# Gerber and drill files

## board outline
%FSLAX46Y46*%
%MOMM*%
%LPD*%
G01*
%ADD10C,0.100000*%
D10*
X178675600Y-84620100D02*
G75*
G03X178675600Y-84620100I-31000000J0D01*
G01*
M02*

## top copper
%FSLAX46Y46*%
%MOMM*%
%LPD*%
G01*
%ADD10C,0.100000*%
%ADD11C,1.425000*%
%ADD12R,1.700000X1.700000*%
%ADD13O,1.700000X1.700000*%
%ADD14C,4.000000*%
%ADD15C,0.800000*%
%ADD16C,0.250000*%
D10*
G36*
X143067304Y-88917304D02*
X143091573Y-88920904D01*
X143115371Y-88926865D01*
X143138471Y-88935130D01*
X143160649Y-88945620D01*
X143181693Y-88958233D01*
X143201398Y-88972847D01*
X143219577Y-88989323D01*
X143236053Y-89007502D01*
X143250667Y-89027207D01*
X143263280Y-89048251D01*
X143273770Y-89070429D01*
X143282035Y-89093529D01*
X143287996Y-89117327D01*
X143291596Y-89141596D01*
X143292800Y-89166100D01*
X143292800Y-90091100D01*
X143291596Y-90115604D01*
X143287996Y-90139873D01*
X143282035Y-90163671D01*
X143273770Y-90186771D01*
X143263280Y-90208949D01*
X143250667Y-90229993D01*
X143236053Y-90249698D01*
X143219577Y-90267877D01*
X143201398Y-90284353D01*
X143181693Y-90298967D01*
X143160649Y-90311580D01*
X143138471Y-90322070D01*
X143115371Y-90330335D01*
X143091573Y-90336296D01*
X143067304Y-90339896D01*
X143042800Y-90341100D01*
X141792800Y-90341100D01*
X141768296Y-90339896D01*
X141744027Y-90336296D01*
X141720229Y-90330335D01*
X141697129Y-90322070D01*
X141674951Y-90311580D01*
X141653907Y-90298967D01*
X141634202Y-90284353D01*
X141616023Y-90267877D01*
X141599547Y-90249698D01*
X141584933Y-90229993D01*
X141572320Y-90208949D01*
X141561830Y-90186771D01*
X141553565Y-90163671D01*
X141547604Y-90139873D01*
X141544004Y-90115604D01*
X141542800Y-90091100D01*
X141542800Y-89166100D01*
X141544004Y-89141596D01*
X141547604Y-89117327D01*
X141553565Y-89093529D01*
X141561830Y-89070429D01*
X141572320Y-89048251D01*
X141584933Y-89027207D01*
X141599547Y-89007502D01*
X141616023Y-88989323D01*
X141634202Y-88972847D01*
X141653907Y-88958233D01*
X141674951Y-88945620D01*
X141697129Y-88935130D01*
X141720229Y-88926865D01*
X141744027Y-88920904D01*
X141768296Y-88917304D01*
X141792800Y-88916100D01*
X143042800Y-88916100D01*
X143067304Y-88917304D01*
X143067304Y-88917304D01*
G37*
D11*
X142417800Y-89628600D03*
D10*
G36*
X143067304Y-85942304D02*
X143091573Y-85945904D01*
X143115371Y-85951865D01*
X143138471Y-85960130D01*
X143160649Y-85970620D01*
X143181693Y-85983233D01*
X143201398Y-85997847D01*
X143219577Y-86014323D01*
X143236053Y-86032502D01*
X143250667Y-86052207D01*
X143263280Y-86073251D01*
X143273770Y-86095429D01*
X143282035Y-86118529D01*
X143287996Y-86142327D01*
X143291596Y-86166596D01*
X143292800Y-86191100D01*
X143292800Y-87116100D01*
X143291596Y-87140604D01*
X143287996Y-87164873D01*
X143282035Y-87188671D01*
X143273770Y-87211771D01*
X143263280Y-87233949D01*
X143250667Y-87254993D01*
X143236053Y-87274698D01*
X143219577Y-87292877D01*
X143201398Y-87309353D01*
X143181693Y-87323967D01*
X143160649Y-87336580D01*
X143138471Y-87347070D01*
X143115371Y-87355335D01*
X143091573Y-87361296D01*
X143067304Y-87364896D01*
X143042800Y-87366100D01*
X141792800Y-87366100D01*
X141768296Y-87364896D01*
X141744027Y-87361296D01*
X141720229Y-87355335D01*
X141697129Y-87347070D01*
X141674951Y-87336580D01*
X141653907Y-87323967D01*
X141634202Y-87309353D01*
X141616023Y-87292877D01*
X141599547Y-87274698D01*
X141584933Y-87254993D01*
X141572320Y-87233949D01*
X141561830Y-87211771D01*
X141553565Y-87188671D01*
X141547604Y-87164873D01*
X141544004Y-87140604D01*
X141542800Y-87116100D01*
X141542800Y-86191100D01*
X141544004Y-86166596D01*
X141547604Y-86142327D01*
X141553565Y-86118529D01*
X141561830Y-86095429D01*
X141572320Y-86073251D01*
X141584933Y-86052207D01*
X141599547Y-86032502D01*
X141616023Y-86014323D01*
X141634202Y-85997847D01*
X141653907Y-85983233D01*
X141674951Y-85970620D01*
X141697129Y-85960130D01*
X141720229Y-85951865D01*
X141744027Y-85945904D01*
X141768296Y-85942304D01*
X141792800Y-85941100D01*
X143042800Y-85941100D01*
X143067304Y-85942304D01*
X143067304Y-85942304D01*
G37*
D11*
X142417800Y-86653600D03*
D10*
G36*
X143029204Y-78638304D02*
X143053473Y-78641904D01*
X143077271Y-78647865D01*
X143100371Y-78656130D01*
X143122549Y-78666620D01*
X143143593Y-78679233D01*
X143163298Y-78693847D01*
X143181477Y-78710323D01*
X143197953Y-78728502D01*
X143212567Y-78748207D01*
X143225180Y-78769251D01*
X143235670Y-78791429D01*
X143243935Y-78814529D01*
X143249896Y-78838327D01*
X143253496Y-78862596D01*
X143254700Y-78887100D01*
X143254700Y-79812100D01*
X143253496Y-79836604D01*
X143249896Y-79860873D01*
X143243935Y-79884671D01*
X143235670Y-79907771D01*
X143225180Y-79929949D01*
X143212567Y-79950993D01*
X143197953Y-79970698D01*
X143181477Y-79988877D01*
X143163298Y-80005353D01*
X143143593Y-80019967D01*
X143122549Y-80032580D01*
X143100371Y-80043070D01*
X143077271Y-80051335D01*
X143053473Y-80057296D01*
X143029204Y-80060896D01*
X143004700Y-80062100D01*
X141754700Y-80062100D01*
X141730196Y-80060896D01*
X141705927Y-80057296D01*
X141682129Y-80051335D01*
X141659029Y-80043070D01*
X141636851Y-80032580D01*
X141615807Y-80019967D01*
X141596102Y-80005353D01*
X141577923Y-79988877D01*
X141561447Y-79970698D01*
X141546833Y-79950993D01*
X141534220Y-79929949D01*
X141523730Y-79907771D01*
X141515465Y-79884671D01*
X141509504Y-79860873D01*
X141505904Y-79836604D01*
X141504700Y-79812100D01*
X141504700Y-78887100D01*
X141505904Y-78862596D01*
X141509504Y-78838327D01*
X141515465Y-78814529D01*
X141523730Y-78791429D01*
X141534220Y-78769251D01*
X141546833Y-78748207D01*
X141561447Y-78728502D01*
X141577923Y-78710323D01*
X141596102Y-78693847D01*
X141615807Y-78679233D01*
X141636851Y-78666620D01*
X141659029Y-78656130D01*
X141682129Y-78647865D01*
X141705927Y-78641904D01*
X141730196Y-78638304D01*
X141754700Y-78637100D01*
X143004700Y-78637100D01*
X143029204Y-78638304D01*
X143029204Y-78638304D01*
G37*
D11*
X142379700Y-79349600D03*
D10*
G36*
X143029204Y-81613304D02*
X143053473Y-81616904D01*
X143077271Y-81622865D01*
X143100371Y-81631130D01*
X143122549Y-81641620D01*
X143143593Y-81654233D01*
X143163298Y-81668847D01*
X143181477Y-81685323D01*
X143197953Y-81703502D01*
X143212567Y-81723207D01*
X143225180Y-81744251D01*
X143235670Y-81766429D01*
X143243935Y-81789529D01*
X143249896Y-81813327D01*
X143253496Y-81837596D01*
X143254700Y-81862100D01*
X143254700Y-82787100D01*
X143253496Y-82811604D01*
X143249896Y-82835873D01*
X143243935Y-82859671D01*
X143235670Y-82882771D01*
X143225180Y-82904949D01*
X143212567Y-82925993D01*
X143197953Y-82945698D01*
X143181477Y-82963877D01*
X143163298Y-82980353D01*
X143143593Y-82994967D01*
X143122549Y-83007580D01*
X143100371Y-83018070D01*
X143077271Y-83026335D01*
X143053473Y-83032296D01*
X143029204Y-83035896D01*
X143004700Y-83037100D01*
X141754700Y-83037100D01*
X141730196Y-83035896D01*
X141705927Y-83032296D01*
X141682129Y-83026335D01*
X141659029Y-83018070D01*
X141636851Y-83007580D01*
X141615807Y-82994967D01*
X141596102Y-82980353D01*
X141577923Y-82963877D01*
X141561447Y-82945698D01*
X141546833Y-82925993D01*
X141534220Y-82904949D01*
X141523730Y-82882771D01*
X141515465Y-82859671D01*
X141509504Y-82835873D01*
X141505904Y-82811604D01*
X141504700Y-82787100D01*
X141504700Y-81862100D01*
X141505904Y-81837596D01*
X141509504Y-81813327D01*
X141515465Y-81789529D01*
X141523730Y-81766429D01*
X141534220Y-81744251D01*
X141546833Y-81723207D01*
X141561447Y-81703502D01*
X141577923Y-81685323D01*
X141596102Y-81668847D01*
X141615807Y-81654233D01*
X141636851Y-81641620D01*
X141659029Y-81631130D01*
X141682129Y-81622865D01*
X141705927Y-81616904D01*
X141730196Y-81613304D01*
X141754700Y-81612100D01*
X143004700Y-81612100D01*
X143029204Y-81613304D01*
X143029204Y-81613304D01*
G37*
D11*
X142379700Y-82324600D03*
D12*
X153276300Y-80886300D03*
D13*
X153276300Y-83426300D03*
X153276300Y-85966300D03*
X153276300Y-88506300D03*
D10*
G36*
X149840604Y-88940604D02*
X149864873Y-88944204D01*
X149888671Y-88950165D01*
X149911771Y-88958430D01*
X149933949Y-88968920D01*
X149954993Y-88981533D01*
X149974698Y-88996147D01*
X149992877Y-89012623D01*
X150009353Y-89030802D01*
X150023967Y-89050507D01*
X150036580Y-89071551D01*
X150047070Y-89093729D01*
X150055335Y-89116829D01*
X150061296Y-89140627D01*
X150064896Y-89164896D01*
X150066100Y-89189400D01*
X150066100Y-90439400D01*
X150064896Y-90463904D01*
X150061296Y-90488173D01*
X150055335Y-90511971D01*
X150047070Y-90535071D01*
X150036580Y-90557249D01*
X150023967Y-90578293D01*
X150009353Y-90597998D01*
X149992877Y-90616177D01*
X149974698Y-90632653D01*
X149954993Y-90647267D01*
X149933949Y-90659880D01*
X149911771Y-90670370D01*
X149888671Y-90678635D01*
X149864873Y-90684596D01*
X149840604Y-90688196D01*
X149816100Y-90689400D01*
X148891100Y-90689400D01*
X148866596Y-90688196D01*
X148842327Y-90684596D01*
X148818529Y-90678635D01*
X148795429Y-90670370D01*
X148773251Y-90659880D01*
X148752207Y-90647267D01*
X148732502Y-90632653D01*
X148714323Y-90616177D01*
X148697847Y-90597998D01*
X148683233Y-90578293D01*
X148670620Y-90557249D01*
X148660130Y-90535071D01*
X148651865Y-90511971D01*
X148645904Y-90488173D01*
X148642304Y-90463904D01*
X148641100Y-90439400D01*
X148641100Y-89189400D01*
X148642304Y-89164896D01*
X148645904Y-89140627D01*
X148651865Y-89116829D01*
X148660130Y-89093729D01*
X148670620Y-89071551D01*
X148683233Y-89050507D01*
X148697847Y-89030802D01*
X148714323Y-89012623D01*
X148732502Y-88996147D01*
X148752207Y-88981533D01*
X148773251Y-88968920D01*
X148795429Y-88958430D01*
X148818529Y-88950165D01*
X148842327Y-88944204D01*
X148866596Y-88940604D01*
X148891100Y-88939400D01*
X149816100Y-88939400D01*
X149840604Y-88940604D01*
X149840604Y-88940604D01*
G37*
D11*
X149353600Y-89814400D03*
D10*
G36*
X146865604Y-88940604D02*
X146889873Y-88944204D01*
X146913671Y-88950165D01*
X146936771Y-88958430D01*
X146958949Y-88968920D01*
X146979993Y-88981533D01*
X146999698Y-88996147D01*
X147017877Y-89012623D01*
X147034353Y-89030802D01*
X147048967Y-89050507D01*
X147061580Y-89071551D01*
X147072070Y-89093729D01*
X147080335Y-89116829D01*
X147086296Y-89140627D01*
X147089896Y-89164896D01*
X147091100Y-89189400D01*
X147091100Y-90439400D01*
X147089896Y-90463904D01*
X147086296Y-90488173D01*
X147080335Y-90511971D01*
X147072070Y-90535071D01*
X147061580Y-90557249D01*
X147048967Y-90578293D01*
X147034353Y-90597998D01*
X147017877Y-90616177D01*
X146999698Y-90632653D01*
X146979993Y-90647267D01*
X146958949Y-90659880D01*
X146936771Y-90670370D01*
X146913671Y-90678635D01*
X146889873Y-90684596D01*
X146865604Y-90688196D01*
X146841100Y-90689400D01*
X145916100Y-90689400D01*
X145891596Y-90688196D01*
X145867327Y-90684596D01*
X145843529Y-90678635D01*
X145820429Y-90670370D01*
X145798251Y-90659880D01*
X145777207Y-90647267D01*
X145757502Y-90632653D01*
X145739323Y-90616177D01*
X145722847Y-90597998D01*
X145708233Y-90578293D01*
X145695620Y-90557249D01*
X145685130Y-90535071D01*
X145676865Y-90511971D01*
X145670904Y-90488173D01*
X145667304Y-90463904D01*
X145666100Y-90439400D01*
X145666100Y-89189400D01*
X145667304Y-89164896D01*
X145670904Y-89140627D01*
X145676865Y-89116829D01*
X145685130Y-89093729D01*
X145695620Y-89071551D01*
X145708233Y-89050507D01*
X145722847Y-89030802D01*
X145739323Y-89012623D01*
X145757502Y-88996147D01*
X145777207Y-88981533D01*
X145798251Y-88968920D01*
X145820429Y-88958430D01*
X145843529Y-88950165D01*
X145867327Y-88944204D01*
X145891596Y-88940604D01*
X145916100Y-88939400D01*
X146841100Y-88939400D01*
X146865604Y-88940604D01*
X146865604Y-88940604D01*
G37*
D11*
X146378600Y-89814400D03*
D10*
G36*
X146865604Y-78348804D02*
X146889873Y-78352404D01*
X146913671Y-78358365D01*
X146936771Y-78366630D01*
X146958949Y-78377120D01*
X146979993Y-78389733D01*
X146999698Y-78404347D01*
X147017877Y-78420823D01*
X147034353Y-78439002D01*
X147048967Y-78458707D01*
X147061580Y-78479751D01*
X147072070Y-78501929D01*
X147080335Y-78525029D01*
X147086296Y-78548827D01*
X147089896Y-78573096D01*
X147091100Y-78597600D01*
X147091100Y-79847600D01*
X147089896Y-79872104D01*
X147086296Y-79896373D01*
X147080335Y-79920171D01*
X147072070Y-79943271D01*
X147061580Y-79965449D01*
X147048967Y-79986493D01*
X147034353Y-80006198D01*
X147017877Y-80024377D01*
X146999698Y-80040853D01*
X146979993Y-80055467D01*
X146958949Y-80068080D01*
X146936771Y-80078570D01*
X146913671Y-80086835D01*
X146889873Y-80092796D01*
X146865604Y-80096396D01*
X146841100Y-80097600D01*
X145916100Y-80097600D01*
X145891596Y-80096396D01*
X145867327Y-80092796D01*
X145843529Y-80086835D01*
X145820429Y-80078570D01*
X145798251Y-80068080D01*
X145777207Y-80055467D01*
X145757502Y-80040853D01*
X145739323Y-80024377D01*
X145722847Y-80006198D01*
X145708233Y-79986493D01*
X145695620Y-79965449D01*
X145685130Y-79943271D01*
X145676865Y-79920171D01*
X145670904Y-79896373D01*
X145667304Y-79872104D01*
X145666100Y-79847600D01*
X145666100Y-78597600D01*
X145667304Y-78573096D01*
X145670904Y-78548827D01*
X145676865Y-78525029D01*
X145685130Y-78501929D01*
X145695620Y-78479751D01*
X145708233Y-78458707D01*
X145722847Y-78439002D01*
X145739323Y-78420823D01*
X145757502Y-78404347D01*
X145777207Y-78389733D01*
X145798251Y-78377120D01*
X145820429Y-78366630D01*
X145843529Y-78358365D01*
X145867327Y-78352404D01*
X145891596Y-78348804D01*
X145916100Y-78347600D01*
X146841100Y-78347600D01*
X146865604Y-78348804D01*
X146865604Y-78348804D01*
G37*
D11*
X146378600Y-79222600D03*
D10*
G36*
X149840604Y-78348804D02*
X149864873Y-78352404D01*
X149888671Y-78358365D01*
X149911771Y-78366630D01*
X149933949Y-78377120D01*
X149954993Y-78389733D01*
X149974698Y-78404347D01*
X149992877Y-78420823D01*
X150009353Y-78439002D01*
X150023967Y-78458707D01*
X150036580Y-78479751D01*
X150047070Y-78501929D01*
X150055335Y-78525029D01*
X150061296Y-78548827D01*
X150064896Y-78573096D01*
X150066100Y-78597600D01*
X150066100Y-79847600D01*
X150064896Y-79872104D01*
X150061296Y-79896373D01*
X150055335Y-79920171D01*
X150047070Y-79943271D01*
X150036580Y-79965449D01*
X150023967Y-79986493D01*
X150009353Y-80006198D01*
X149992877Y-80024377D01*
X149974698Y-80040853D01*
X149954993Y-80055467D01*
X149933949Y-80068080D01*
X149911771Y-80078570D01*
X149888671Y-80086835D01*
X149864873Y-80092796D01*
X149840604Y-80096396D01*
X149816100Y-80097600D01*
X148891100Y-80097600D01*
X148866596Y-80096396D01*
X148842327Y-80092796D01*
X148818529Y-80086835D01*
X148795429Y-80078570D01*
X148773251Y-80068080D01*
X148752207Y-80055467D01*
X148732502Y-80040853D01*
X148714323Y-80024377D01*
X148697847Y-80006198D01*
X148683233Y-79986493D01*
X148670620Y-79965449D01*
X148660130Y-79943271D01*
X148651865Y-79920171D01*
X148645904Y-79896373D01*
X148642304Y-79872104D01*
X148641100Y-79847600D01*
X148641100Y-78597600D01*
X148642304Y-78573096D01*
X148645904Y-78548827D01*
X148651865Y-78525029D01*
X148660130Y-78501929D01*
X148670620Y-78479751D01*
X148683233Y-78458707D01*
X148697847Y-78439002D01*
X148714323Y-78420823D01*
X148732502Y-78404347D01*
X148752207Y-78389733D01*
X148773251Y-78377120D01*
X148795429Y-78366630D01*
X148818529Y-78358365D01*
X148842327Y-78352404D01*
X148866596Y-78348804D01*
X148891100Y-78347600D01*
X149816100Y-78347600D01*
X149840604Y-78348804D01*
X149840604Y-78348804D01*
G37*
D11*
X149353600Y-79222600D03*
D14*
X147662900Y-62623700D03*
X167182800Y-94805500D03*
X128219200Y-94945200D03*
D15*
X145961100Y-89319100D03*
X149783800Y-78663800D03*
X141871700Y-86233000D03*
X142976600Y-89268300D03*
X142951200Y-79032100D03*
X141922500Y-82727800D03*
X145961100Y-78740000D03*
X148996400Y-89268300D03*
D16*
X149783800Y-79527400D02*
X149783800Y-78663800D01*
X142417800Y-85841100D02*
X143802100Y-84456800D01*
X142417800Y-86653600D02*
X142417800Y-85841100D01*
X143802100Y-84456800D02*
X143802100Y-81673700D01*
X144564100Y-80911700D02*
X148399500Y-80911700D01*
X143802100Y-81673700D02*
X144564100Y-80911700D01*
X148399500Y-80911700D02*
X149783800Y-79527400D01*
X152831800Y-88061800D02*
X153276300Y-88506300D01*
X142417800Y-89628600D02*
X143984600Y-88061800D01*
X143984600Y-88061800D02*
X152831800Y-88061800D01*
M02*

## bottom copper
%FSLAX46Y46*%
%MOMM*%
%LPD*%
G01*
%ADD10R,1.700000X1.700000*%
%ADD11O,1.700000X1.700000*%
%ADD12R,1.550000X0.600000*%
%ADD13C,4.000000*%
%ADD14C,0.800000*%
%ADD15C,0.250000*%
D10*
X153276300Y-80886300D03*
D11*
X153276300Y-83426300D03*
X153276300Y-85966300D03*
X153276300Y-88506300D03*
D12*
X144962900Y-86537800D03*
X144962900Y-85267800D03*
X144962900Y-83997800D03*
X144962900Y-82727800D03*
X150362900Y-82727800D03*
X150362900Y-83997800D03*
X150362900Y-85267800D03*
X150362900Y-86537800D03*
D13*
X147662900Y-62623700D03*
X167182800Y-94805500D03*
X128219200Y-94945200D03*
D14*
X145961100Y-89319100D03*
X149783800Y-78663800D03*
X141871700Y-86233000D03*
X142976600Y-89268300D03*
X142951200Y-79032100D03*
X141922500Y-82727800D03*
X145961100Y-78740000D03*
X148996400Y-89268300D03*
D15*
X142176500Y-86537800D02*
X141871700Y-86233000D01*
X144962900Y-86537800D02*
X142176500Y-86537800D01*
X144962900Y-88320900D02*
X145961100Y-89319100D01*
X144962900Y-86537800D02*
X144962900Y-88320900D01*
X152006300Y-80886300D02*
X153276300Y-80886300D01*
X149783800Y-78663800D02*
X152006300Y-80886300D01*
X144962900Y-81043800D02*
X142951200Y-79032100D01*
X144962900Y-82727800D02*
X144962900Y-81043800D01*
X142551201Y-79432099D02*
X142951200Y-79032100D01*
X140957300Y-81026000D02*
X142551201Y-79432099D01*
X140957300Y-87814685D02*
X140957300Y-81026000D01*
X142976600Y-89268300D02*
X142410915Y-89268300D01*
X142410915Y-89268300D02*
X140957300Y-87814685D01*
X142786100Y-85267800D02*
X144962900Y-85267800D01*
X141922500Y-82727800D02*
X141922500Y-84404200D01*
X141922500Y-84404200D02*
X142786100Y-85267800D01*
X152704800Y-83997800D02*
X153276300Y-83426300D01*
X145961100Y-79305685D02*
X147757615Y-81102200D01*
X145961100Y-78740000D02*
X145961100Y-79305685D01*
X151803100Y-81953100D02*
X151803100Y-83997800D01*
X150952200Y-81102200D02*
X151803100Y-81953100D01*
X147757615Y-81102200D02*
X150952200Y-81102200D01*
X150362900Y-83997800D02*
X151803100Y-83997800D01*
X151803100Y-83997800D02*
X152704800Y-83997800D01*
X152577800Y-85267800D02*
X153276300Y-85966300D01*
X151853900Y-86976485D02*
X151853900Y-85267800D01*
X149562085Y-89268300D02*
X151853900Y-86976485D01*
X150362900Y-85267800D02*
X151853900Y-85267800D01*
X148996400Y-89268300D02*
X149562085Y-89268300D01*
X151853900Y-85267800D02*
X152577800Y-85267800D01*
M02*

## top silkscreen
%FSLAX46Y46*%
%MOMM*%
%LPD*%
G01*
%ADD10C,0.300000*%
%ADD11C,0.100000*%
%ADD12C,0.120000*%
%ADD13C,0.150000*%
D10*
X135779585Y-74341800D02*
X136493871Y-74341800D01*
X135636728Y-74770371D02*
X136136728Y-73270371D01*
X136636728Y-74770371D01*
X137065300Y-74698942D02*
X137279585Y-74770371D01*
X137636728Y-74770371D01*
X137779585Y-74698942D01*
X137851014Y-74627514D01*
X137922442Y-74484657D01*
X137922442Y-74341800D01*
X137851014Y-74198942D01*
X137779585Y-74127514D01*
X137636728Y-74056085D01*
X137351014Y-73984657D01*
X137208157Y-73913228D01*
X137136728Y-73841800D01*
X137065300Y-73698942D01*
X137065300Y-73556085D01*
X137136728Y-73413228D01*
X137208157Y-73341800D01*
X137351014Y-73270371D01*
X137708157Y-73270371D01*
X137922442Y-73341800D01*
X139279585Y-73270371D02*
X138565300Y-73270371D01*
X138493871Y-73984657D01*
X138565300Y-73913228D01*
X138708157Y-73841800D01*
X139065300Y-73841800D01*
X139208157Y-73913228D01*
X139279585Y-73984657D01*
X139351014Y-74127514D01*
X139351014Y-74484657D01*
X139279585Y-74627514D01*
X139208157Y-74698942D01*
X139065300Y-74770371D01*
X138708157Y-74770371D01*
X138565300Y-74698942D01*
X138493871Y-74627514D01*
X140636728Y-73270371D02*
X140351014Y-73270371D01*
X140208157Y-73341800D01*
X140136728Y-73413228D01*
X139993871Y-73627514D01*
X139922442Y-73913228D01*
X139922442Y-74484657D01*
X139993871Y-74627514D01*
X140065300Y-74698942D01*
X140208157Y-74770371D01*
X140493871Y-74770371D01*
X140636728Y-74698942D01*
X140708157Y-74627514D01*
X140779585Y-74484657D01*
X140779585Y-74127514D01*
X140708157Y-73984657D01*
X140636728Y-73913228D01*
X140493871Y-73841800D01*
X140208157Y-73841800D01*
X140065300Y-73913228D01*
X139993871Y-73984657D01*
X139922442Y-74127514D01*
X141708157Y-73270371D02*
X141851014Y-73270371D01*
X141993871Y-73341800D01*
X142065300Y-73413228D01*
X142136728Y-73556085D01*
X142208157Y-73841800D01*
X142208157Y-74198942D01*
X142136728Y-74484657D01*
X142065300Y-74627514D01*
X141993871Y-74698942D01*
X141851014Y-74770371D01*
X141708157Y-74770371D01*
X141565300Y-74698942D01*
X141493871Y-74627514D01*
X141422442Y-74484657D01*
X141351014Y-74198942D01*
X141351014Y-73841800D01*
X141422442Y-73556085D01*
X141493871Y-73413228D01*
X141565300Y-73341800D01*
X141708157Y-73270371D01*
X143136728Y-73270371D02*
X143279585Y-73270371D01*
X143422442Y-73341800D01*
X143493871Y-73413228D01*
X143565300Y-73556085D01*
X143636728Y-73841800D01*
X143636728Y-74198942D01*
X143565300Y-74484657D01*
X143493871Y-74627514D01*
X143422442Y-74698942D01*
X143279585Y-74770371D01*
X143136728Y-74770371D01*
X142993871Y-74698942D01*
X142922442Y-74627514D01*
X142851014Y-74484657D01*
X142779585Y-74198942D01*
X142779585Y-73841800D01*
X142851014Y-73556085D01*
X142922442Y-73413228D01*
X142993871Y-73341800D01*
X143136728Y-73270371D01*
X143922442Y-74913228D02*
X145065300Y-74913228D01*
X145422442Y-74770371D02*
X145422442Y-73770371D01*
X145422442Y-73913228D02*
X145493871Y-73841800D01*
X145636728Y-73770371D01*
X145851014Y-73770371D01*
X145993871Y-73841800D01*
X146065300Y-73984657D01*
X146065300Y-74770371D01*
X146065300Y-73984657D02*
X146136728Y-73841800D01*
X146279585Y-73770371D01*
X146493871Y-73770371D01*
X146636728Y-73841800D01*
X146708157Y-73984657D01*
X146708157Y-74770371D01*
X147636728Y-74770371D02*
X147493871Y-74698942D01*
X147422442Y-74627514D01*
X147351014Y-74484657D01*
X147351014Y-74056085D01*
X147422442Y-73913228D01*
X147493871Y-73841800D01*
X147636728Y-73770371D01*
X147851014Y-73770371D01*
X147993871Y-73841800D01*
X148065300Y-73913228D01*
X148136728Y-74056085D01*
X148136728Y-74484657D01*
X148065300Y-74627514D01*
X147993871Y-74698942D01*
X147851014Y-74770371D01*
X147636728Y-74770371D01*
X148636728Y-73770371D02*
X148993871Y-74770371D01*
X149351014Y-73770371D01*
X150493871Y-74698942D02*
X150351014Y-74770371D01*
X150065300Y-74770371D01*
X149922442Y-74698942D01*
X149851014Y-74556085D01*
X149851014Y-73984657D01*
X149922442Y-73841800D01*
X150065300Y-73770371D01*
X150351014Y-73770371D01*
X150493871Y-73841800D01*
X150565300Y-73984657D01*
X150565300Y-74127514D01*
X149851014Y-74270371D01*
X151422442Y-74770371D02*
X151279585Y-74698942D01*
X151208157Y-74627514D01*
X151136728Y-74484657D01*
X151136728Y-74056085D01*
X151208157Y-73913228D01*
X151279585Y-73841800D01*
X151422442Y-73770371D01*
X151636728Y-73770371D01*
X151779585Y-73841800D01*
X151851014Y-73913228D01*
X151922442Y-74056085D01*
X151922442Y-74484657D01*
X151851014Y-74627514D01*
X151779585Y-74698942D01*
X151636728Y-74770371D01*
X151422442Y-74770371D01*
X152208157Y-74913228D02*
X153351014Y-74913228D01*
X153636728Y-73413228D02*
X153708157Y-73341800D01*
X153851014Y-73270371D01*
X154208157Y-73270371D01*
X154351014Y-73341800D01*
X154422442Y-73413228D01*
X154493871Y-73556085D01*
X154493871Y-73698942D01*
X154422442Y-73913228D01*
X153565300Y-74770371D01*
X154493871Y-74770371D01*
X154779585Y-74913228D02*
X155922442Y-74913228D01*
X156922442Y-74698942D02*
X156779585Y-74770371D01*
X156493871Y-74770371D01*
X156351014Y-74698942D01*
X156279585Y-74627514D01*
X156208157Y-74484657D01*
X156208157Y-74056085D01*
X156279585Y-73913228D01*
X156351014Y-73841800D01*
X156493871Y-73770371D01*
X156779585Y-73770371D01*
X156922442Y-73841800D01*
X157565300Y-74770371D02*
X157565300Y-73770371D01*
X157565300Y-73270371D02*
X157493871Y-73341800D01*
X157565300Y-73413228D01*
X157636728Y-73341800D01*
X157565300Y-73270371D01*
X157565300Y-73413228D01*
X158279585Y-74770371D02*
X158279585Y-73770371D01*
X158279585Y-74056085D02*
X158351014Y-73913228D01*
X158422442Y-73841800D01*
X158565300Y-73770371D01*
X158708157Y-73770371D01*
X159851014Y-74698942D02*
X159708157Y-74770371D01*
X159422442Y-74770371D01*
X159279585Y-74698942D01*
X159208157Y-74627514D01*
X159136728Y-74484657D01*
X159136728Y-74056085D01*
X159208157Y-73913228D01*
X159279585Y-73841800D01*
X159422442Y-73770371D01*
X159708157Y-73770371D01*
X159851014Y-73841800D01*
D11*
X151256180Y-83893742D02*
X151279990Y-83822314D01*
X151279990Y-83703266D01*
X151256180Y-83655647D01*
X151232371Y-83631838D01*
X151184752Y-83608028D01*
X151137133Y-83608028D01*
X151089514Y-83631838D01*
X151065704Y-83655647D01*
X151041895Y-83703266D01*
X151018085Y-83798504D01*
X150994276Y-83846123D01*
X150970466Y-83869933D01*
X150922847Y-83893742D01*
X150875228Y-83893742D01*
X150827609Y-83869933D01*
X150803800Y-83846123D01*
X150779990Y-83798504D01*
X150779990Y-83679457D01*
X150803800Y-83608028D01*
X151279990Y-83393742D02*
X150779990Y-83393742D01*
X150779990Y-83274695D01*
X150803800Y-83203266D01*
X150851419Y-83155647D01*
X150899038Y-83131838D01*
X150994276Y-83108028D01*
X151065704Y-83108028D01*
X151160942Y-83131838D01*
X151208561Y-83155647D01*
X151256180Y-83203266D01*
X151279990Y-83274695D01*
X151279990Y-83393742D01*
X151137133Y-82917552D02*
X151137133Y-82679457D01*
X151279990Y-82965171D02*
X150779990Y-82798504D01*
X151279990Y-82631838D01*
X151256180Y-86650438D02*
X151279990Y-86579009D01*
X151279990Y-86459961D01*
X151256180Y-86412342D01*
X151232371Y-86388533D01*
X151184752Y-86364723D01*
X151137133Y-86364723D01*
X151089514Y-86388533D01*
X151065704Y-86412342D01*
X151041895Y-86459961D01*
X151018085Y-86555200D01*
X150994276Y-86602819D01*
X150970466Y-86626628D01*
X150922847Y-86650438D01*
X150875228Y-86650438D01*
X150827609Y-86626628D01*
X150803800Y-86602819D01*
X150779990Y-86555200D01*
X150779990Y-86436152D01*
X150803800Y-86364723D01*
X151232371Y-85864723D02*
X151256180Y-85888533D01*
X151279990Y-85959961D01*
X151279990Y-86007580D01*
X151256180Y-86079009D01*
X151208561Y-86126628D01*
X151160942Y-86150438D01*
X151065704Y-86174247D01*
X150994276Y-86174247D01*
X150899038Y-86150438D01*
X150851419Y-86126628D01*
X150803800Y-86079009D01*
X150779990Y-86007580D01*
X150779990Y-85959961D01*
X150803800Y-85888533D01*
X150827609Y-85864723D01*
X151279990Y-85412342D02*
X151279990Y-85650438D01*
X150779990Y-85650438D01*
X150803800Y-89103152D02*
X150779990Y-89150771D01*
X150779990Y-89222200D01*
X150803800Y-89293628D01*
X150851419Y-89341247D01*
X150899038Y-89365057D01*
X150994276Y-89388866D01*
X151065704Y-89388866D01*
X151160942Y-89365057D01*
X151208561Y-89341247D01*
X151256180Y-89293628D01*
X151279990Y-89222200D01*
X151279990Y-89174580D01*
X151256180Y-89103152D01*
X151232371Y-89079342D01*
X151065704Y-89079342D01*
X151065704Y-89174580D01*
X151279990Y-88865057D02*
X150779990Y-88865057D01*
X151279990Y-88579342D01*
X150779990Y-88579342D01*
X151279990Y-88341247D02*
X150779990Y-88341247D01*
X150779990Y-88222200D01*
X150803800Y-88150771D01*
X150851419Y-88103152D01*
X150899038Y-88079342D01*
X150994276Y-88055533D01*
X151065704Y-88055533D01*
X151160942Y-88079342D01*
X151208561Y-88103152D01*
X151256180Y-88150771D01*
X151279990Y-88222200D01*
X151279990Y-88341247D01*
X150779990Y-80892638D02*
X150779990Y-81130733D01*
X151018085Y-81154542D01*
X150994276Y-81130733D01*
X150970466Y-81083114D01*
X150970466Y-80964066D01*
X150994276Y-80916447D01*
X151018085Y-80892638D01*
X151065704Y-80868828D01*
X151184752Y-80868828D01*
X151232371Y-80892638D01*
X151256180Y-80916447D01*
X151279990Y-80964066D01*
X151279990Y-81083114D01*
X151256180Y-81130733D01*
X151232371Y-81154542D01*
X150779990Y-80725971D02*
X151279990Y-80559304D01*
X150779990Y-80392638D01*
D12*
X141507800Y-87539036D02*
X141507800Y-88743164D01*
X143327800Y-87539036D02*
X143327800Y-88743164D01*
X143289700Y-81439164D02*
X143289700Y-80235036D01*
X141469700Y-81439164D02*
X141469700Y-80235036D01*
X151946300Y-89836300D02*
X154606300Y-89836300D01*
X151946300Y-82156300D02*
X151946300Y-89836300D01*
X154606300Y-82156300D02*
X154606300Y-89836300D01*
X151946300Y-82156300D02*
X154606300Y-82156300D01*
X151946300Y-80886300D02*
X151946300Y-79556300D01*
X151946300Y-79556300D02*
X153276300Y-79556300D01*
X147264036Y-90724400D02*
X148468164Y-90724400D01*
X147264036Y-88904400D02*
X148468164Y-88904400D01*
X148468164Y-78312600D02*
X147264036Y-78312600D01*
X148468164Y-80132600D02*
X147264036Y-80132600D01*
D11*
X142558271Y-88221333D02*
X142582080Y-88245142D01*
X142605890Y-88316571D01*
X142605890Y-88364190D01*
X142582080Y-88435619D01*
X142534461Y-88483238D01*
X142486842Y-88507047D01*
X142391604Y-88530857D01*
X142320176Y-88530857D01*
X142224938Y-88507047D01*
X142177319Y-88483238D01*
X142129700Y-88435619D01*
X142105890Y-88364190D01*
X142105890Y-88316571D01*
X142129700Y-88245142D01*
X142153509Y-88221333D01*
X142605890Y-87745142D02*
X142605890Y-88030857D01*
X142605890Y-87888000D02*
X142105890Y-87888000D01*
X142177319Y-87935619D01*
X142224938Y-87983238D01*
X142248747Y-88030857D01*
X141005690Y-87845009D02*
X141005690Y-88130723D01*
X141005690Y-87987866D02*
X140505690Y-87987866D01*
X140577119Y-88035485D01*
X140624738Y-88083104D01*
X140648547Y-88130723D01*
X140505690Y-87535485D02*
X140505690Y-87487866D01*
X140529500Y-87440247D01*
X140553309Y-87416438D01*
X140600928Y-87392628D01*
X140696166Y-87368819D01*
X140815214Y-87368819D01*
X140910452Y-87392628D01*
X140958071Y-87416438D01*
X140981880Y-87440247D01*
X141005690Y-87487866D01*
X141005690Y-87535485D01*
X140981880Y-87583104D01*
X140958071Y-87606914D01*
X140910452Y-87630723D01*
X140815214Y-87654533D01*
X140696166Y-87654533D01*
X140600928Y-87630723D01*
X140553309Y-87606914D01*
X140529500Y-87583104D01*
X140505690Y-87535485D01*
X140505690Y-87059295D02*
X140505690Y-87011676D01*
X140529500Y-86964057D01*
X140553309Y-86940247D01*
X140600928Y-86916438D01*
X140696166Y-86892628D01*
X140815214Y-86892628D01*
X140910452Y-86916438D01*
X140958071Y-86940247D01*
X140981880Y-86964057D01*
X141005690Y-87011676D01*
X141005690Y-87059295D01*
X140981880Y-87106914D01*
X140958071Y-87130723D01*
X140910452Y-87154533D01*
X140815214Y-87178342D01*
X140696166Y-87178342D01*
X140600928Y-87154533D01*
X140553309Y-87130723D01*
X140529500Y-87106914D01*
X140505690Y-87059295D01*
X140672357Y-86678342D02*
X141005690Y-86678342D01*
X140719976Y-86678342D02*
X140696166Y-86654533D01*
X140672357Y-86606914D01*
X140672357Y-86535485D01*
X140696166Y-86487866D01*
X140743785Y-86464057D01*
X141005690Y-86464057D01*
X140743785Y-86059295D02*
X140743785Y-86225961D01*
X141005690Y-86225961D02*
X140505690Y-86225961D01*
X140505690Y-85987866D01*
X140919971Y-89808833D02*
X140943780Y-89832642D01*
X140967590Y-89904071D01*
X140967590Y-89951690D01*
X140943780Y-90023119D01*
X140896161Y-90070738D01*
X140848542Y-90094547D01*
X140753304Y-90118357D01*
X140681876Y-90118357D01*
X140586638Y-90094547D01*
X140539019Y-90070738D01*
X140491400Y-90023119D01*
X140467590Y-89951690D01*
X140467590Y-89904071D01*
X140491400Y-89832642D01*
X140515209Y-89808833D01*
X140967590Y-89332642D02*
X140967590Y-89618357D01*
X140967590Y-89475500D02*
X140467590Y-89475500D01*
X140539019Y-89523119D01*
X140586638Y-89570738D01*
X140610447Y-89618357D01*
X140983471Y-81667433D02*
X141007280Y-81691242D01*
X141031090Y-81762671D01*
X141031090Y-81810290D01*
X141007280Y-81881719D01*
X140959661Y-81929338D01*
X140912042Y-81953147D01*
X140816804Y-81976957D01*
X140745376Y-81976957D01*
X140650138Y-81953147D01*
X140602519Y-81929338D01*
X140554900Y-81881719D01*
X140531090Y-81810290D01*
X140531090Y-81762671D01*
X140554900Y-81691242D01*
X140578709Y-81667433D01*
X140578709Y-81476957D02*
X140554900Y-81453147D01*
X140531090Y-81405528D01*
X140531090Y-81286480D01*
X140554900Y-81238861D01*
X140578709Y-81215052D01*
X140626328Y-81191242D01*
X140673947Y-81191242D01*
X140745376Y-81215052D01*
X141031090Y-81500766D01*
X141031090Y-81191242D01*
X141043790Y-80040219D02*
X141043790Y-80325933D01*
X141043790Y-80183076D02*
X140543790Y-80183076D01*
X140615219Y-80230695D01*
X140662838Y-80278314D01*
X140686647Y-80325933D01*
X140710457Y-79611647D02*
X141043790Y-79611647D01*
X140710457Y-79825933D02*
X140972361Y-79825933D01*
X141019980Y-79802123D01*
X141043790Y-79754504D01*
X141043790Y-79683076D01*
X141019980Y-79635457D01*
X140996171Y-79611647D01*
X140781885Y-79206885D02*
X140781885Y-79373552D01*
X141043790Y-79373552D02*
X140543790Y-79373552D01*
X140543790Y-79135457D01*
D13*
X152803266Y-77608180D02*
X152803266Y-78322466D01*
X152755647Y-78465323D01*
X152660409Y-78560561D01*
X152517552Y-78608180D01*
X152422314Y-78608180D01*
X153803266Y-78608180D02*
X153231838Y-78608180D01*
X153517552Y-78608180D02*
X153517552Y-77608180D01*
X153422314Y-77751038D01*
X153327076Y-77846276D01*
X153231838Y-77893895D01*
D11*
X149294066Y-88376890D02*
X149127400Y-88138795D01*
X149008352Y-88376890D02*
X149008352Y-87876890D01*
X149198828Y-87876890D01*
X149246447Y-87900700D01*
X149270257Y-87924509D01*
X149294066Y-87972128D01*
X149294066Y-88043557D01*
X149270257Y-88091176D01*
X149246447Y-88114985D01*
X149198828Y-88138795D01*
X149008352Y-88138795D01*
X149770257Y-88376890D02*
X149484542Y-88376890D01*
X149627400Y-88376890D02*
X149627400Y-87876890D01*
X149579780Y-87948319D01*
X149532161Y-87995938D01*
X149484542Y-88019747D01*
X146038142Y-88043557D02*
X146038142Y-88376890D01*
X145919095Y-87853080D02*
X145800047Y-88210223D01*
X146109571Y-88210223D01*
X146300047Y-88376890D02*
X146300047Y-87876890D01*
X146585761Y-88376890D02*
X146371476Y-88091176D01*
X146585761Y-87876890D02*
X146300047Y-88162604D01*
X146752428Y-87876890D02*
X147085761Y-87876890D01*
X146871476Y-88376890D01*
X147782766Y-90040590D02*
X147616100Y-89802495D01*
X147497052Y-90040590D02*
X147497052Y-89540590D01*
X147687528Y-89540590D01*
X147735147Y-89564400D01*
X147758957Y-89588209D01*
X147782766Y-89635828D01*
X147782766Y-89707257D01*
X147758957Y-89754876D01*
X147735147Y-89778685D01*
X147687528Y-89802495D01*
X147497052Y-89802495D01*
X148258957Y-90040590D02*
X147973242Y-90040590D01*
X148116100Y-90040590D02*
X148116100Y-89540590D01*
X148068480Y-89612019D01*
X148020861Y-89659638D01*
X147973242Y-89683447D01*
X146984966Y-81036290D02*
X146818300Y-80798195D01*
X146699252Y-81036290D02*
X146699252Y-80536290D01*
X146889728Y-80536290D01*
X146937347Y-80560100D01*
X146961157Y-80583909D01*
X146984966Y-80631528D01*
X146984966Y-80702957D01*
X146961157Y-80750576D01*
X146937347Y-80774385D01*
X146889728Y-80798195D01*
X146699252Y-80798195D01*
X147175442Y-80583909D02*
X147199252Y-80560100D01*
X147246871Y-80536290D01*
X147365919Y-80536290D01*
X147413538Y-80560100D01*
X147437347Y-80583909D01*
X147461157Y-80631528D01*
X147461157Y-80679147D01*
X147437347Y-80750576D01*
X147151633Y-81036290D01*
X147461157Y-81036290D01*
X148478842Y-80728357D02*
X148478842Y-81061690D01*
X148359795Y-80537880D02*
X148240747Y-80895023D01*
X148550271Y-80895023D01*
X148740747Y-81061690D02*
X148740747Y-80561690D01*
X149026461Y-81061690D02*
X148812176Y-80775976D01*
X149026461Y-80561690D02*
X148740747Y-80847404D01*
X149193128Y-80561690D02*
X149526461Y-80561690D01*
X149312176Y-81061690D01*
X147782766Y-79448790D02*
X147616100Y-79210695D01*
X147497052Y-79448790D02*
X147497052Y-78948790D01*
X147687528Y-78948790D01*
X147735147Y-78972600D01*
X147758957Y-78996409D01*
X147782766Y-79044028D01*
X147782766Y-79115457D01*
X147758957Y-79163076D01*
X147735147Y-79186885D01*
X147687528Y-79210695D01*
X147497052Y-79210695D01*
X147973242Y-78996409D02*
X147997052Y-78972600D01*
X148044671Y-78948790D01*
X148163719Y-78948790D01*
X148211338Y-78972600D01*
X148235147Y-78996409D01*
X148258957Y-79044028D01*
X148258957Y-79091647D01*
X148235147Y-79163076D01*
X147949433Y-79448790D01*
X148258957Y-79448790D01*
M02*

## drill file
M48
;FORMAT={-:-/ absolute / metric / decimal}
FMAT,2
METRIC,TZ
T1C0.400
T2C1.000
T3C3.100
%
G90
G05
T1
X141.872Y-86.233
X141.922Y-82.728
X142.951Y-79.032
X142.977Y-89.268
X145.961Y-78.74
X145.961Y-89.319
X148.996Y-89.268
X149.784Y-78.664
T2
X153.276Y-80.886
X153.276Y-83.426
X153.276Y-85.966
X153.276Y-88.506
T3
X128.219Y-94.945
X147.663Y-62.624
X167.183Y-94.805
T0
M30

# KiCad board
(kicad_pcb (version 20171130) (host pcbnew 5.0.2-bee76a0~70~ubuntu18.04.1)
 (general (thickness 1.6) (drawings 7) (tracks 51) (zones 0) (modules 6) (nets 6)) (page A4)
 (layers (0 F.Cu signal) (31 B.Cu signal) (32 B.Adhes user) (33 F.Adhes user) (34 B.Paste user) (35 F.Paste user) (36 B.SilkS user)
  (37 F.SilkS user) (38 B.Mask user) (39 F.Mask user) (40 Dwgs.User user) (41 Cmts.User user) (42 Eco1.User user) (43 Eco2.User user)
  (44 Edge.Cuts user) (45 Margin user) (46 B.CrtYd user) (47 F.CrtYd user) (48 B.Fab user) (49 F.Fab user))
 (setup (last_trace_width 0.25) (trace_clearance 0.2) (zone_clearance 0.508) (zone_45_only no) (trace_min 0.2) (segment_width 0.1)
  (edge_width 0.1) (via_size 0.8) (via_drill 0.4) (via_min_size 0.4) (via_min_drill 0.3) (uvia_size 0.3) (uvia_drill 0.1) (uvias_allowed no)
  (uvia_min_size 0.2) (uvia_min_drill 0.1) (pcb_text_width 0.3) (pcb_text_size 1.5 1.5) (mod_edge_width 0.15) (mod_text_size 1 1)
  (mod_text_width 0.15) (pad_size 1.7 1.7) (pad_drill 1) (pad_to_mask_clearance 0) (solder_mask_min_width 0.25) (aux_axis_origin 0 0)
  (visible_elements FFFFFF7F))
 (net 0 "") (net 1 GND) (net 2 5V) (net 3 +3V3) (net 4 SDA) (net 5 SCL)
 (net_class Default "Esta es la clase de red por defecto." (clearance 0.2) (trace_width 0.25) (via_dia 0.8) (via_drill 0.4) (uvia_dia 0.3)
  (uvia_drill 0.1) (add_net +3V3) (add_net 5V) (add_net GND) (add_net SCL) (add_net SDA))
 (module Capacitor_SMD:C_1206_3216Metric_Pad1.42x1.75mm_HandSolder (layer F.Cu) (at 142.4178 88.1411 270)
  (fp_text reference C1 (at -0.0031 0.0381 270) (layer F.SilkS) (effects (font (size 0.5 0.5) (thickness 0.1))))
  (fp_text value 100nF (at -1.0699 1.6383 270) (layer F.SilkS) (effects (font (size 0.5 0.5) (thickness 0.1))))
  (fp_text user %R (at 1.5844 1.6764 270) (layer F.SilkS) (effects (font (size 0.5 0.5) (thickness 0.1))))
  (fp_line (start -0.602064 0.91) (end 0.602064 0.91) (layer F.SilkS) (width 0.12))
  (fp_line (start -0.602064 -0.91) (end 0.602064 -0.91) (layer F.SilkS) (width 0.12))
  (pad 2 smd roundrect (at 1.4875 0 270) (size 1.425 1.75) (layers F.Cu F.Paste F.Mask) (roundrect_rratio 0.175439) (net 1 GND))
  (pad 1 smd roundrect (at -1.4875 0 270) (size 1.425 1.75) (layers F.Cu F.Paste F.Mask) (roundrect_rratio 0.175439) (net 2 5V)))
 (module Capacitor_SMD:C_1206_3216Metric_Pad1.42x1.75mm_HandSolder (layer F.Cu) (at 142.3797 80.8371 90)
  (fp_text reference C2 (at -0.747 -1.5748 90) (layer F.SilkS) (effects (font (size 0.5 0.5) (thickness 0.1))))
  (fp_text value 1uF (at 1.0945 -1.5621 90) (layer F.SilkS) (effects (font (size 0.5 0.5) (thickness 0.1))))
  (fp_line (start -0.602064 0.91) (end 0.602064 0.91) (layer F.SilkS) (width 0.12))
  (fp_line (start -0.602064 -0.91) (end 0.602064 -0.91) (layer F.SilkS) (width 0.12))
  (pad 2 smd roundrect (at 1.4875 0 90) (size 1.425 1.75) (layers F.Cu F.Paste F.Mask) (roundrect_rratio 0.175439) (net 1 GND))
  (pad 1 smd roundrect (at -1.4875 0 90) (size 1.425 1.75) (layers F.Cu F.Paste F.Mask) (roundrect_rratio 0.175439) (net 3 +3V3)))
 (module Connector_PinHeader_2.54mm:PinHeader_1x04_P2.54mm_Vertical (layer F.Cu) (at 153.2763 80.8863)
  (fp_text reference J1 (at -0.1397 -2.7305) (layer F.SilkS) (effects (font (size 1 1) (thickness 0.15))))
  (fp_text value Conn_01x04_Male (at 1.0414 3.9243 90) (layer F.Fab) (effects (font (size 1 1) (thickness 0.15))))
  (fp_line (start -1.33 8.95) (end 1.33 8.95) (layer F.SilkS) (width 0.12))
  (fp_line (start -1.33 1.27) (end -1.33 8.95) (layer F.SilkS) (width 0.12))
  (fp_line (start 1.33 1.27) (end 1.33 8.95) (layer F.SilkS) (width 0.12))
  (fp_line (start -1.33 1.27) (end 1.33 1.27) (layer F.SilkS) (width 0.12))
  (fp_line (start -1.33 0) (end -1.33 -1.33) (layer F.SilkS) (width 0.12))
  (fp_line (start -1.33 -1.33) (end 0 -1.33) (layer F.SilkS) (width 0.12))
  (pad 1 thru_hole rect (at 0 0) (size 1.7 1.7) (drill 1) (layers *.Cu *.Mask) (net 2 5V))
  (pad 2 thru_hole oval (at 0 2.54) (size 1.7 1.7) (drill 1) (layers *.Cu *.Mask) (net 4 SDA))
  (pad 3 thru_hole oval (at 0 5.08) (size 1.7 1.7) (drill 1) (layers *.Cu *.Mask) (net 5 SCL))
  (pad 4 thru_hole oval (at 0 7.62) (size 1.7 1.7) (drill 1) (layers *.Cu *.Mask) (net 1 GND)))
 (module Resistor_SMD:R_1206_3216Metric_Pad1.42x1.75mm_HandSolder (layer F.Cu) (at 147.8661 89.8144)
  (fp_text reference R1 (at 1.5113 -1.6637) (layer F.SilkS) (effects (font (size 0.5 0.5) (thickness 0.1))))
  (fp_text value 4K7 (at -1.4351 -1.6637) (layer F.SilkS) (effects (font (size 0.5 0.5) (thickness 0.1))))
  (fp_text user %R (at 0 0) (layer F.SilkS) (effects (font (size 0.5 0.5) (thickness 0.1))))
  (fp_line (start -0.602064 0.91) (end 0.602064 0.91) (layer F.SilkS) (width 0.12))
  (fp_line (start -0.602064 -0.91) (end 0.602064 -0.91) (layer F.SilkS) (width 0.12))
  (pad 2 smd roundrect (at 1.4875 0) (size 1.425 1.75) (layers F.Cu F.Paste F.Mask) (roundrect_rratio 0.175439) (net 5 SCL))
  (pad 1 smd roundrect (at -1.4875 0) (size 1.425 1.75) (layers F.Cu F.Paste F.Mask) (roundrect_rratio 0.175439) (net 2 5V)))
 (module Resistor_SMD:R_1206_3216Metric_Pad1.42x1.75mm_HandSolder (layer F.Cu) (at 147.8661 79.2226 180)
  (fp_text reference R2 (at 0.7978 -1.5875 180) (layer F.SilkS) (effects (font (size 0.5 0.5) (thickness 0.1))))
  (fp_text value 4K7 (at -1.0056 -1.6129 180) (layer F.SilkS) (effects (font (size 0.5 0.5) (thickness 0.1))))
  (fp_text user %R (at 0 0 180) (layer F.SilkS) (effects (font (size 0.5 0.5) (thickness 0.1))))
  (fp_line (start -0.602064 0.91) (end 0.602064 0.91) (layer F.SilkS) (width 0.12))
  (fp_line (start -0.602064 -0.91) (end 0.602064 -0.91) (layer F.SilkS) (width 0.12))
  (pad 2 smd roundrect (at 1.4875 0 180) (size 1.425 1.75) (layers F.Cu F.Paste F.Mask) (roundrect_rratio 0.175439) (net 4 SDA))
  (pad 1 smd roundrect (at -1.4875 0 180) (size 1.425 1.75) (layers F.Cu F.Paste F.Mask) (roundrect_rratio 0.175439) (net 2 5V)))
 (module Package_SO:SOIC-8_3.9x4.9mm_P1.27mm (layer B.Cu) (at 147.6629 84.6328)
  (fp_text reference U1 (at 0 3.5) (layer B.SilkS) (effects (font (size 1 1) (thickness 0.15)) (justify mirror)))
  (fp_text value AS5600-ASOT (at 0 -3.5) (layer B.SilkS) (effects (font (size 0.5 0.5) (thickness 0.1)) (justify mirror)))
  (pad 1 smd rect (at -2.7 1.905) (size 1.55 0.6) (layers B.Cu B.Paste B.Mask) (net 2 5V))
  (pad 2 smd rect (at -2.7 0.635) (size 1.55 0.6) (layers B.Cu B.Paste B.Mask) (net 3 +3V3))
  (pad 3 smd rect (at -2.7 -0.635) (size 1.55 0.6) (layers B.Cu B.Paste B.Mask))
  (pad 4 smd rect (at -2.7 -1.905) (size 1.55 0.6) (layers B.Cu B.Paste B.Mask) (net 1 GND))
  (pad 5 smd rect (at 2.7 -1.905) (size 1.55 0.6) (layers B.Cu B.Paste B.Mask))
  (pad 6 smd rect (at 2.7 -0.635) (size 1.55 0.6) (layers B.Cu B.Paste B.Mask) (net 4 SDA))
  (pad 7 smd rect (at 2.7 0.635) (size 1.55 0.6) (layers B.Cu B.Paste B.Mask) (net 5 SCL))
  (pad 8 smd rect (at 2.7 1.905) (size 1.55 0.6) (layers B.Cu B.Paste B.Mask)))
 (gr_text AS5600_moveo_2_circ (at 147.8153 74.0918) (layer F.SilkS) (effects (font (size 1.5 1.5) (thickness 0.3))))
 (gr_circle (center 147.6756 84.6201) (end 178.6756 84.6201) (layer Edge.Cuts) (width 0.1))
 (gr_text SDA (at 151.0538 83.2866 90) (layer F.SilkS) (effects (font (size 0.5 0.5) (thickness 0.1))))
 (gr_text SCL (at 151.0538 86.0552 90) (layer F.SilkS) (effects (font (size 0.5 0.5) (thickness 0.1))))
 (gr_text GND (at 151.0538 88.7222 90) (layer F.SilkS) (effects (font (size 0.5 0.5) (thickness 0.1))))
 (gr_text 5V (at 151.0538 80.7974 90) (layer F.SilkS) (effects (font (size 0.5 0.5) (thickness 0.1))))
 (via (at 147.6629 62.6237) (size 4) (drill 3.1) (layers F.Cu B.Cu) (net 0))
 (via (at 167.1828 94.8055) (size 4) (drill 3.1) (layers F.Cu B.Cu) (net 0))
 (via (at 128.2192 94.9452) (size 4) (drill 3.1) (layers F.Cu B.Cu) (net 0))
 (via (at 145.9611 89.3191) (size 0.8) (drill 0.4) (layers F.Cu B.Cu) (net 2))
 (via (at 149.7838 78.6638) (size 0.8) (drill 0.4) (layers F.Cu B.Cu) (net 2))
 (via (at 141.8717 86.233) (size 0.8) (drill 0.4) (layers F.Cu B.Cu) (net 2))
 (segment (start 142.1765 86.5378) (end 141.8717 86.233) (width 0.25) (layer B.Cu) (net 2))
 (segment (start 144.9629 86.5378) (end 142.1765 86.5378) (width 0.25) (layer B.Cu) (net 2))
 (segment (start 144.9629 88.3209) (end 145.9611 89.3191) (width 0.25) (layer B.Cu) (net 2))
 (segment (start 144.9629 86.5378) (end 144.9629 88.3209) (width 0.25) (layer B.Cu) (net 2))
 (segment (start 152.0063 80.8863) (end 153.2763 80.8863) (width 0.25) (layer B.Cu) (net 2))
 (segment (start 149.7838 78.6638) (end 152.0063 80.8863) (width 0.25) (layer B.Cu) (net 2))
 (segment (start 149.7838 79.5274) (end 149.7838 78.6638) (width 0.25) (layer F.Cu) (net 2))
 (segment (start 142.4178 85.8411) (end 143.8021 84.4568) (width 0.25) (layer F.Cu) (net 2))
 (segment (start 142.4178 86.6536) (end 142.4178 85.8411) (width 0.25) (layer F.Cu) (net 2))
 (segment (start 143.8021 84.4568) (end 143.8021 81.6737) (width 0.25) (layer F.Cu) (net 2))
 (segment (start 144.5641 80.9117) (end 148.3995 80.9117) (width 0.25) (layer F.Cu) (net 2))
 (segment (start 143.8021 81.6737) (end 144.5641 80.9117) (width 0.25) (layer F.Cu) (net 2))
 (segment (start 148.3995 80.9117) (end 149.7838 79.5274) (width 0.25) (layer F.Cu) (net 2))
 (via (at 142.9766 89.2683) (size 0.8) (drill 0.4) (layers F.Cu B.Cu) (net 1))
 (via (at 142.9512 79.0321) (size 0.8) (drill 0.4) (layers F.Cu B.Cu) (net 1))
 (segment (start 144.9629 81.0438) (end 142.9512 79.0321) (width 0.25) (layer B.Cu) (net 1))
 (segment (start 144.9629 82.7278) (end 144.9629 81.0438) (width 0.25) (layer B.Cu) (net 1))
 (segment (start 152.8318 88.0618) (end 153.2763 88.5063) (width 0.25) (layer F.Cu) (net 1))
 (segment (start 142.4178 89.6286) (end 143.9846 88.0618) (width 0.25) (layer F.Cu) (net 1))
 (segment (start 143.9846 88.0618) (end 152.8318 88.0618) (width 0.25) (layer F.Cu) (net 1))
 (segment (start 142.551201 79.432099) (end 142.9512 79.0321) (width 0.25) (layer B.Cu) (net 1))
 (segment (start 140.9573 81.026) (end 142.551201 79.432099) (width 0.25) (layer B.Cu) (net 1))
 (segment (start 140.9573 87.814685) (end 140.9573 81.026) (width 0.25) (layer B.Cu) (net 1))
 (segment (start 142.9766 89.2683) (end 142.410915 89.2683) (width 0.25) (layer B.Cu) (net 1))
 (segment (start 142.410915 89.2683) (end 140.9573 87.814685) (width 0.25) (layer B.Cu) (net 1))
 (via (at 141.9225 82.7278) (size 0.8) (drill 0.4) (layers F.Cu B.Cu) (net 3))
 (segment (start 142.7861 85.2678) (end 144.9629 85.2678) (width 0.25) (layer B.Cu) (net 3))
 (segment (start 141.9225 82.7278) (end 141.9225 84.4042) (width 0.25) (layer B.Cu) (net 3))
 (segment (start 141.9225 84.4042) (end 142.7861 85.2678) (width 0.25) (layer B.Cu) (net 3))
 (via (at 145.9611 78.74) (size 0.8) (drill 0.4) (layers F.Cu B.Cu) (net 4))
 (segment (start 152.7048 83.9978) (end 153.2763 83.4263) (width 0.25) (layer B.Cu) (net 4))
 (segment (start 145.9611 79.305685) (end 147.757615 81.1022) (width 0.25) (layer B.Cu) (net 4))
 (segment (start 145.9611 78.74) (end 145.9611 79.305685) (width 0.25) (layer B.Cu) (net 4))
 (segment (start 151.8031 81.9531) (end 151.8031 83.9978) (width 0.25) (layer B.Cu) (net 4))
 (segment (start 150.9522 81.1022) (end 151.8031 81.9531) (width 0.25) (layer B.Cu) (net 4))
 (segment (start 147.757615 81.1022) (end 150.9522 81.1022) (width 0.25) (layer B.Cu) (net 4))
 (segment (start 150.3629 83.9978) (end 151.8031 83.9978) (width 0.25) (layer B.Cu) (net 4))
 (segment (start 151.8031 83.9978) (end 152.7048 83.9978) (width 0.25) (layer B.Cu) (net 4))
 (via (at 148.9964 89.2683) (size 0.8) (drill 0.4) (layers F.Cu B.Cu) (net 5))
 (segment (start 152.5778 85.2678) (end 153.2763 85.9663) (width 0.25) (layer B.Cu) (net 5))
 (segment (start 151.8539 86.976485) (end 151.8539 85.2678) (width 0.25) (layer B.Cu) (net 5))
 (segment (start 149.562085 89.2683) (end 151.8539 86.976485) (width 0.25) (layer B.Cu) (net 5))
 (segment (start 150.3629 85.2678) (end 151.8539 85.2678) (width 0.25) (layer B.Cu) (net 5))
 (segment (start 148.9964 89.2683) (end 149.562085 89.2683) (width 0.25) (layer B.Cu) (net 5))
 (segment (start 151.8539 85.2678) (end 152.5778 85.2678) (width 0.25) (layer B.Cu) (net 5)))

